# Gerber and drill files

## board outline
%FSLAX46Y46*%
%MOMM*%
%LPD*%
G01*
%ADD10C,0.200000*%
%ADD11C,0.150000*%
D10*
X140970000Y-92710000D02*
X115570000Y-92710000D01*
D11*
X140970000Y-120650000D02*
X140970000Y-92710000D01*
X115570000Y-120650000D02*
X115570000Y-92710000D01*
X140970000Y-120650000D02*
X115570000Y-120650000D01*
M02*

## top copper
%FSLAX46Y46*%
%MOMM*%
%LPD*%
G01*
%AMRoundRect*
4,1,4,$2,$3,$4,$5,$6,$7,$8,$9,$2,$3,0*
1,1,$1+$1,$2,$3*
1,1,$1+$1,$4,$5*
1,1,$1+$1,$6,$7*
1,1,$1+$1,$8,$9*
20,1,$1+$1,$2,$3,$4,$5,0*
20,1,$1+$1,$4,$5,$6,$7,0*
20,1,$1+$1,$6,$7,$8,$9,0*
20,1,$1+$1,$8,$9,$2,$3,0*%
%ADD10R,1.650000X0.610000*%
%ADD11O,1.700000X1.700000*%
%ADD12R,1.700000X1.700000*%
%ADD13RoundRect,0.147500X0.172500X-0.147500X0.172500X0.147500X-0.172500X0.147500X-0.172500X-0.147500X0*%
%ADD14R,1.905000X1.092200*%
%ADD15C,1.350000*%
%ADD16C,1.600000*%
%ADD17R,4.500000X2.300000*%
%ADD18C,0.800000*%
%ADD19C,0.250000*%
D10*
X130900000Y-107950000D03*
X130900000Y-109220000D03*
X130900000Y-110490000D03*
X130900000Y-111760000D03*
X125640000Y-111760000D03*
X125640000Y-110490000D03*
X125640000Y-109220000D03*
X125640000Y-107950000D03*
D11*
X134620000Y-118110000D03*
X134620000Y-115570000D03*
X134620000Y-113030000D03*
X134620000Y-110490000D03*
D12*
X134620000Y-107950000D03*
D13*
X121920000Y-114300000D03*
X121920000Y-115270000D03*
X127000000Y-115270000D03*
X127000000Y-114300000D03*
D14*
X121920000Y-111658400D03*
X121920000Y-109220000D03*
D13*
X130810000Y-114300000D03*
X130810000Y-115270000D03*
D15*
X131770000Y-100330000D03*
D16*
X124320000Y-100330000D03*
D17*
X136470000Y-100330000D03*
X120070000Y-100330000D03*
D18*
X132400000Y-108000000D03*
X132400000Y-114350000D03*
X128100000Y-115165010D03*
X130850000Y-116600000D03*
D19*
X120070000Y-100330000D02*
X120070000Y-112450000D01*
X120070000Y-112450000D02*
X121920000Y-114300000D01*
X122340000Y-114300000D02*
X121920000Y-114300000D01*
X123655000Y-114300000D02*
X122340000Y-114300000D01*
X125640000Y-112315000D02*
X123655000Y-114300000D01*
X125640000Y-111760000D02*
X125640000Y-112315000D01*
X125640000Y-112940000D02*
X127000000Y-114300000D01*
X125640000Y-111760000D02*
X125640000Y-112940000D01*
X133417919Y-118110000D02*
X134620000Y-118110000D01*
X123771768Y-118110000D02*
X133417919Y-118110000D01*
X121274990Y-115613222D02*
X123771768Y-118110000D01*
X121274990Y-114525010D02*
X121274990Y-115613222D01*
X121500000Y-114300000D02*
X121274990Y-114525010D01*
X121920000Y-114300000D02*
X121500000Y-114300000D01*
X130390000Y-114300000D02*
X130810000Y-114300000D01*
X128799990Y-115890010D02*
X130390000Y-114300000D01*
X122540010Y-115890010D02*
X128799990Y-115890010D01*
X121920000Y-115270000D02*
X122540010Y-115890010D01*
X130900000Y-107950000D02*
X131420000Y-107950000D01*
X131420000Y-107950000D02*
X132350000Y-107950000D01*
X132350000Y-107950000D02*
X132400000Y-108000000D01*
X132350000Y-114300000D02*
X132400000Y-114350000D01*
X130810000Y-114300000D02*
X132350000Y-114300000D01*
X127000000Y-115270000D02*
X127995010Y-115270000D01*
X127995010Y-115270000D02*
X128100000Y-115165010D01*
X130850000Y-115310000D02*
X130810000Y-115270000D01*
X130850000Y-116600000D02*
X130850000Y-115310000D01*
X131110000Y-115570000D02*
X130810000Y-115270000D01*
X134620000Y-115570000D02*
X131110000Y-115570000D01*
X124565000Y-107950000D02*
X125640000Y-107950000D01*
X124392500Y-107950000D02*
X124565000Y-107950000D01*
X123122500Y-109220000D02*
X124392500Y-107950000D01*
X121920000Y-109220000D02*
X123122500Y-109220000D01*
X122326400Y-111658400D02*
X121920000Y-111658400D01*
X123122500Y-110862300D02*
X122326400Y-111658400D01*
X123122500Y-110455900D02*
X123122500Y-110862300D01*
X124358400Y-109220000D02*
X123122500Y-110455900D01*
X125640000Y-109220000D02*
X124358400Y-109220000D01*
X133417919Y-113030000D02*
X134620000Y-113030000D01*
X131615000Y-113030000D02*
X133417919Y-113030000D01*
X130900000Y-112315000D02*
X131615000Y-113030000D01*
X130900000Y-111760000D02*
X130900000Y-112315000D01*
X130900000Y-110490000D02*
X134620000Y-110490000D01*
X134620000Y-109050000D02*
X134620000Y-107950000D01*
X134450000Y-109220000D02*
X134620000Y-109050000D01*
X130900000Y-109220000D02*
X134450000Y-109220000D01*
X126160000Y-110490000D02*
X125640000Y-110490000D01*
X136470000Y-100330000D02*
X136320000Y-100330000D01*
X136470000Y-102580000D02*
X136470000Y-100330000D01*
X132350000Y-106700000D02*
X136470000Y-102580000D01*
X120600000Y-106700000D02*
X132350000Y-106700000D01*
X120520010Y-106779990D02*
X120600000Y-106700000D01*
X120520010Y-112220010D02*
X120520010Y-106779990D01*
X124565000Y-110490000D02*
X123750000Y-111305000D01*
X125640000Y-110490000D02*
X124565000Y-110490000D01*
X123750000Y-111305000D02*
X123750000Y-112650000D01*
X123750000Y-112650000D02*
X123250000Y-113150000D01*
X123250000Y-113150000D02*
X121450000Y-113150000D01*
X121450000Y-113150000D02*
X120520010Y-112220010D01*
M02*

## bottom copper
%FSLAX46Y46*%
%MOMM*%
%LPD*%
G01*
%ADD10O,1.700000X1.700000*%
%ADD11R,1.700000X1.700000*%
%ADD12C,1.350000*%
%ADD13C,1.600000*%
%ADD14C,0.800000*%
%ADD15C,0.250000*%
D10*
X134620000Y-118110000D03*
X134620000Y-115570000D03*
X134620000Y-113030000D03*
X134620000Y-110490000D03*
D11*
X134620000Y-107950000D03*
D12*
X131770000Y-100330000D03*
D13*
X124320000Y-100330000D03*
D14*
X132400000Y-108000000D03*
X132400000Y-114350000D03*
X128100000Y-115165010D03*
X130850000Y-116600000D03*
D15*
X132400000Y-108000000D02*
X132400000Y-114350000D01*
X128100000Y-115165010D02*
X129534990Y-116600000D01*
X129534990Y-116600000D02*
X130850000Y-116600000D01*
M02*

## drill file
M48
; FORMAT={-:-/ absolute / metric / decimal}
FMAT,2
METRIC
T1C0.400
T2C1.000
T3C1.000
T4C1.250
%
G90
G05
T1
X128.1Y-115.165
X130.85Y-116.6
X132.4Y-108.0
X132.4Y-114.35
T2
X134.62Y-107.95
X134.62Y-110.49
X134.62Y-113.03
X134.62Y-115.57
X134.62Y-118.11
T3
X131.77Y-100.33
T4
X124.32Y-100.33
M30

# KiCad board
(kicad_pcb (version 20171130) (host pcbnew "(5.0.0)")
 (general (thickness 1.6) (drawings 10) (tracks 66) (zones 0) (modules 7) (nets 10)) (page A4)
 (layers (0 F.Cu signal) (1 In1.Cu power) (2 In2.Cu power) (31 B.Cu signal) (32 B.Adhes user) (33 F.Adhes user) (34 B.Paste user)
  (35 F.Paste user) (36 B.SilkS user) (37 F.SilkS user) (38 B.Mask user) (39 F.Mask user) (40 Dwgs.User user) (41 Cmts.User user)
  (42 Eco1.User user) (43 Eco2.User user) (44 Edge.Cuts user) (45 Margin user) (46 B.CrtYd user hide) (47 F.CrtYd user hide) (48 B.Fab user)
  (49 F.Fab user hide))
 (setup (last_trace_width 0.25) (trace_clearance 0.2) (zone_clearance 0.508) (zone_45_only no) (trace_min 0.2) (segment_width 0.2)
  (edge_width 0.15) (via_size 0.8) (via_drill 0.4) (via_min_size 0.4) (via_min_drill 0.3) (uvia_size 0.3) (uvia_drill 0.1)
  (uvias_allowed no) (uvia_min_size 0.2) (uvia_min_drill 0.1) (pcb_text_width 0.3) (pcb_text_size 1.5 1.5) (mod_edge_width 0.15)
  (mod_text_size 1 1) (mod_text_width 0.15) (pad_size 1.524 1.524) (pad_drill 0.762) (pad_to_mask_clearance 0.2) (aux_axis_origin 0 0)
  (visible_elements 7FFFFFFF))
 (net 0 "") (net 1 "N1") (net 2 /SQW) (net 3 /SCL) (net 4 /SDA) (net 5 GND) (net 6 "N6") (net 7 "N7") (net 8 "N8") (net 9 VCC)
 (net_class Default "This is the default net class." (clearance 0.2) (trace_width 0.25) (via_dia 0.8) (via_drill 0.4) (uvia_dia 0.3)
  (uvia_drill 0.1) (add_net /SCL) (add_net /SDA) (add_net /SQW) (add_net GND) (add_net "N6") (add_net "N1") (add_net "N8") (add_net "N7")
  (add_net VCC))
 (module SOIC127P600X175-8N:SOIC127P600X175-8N (layer F.Cu) (at 128.27 109.855)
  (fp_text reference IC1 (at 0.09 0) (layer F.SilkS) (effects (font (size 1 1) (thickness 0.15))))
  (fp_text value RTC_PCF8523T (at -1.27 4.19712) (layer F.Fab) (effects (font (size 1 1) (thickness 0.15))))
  (pad 8 smd rect (at 2.63 -1.905) (size 1.65 0.61) (layers F.Cu F.Paste F.Mask) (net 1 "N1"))
  (pad 7 smd rect (at 2.63 -0.635) (size 1.65 0.61) (layers F.Cu F.Paste F.Mask) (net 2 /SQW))
  (pad 6 smd rect (at 2.63 0.635) (size 1.65 0.61) (layers F.Cu F.Paste F.Mask) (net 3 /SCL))
  (pad 5 smd rect (at 2.63 1.905) (size 1.65 0.61) (layers F.Cu F.Paste F.Mask) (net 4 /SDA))
  (pad 4 smd rect (at -2.63 1.905) (size 1.65 0.61) (layers F.Cu F.Paste F.Mask) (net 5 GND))
  (pad 3 smd rect (at -2.63 0.635) (size 1.65 0.61) (layers F.Cu F.Paste F.Mask) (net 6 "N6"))
  (pad 2 smd rect (at -2.63 -0.635) (size 1.65 0.61) (layers F.Cu F.Paste F.Mask) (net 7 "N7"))
  (pad 1 smd rect (at -2.63 -1.905) (size 1.65 0.61) (layers F.Cu F.Paste F.Mask) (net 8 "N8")))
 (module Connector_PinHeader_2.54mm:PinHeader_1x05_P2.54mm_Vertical (layer F.Cu) (at 134.62 107.95)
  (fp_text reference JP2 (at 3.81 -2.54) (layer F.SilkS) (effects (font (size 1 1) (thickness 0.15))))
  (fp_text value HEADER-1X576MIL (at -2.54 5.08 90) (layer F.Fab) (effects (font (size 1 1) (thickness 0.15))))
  (pad 5 thru_hole oval (at 0 10.16) (size 1.7 1.7) (drill 1) (layers *.Cu *.Mask) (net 5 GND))
  (pad 4 thru_hole oval (at 0 7.62) (size 1.7 1.7) (drill 1) (layers *.Cu *.Mask) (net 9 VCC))
  (pad 3 thru_hole oval (at 0 5.08) (size 1.7 1.7) (drill 1) (layers *.Cu *.Mask) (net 4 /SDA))
  (pad 2 thru_hole oval (at 0 2.54) (size 1.7 1.7) (drill 1) (layers *.Cu *.Mask) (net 3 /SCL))
  (pad 1 thru_hole rect (at 0 0) (size 1.7 1.7) (drill 1) (layers *.Cu *.Mask) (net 2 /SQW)))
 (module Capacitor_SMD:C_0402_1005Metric (layer F.Cu) (at 121.92 114.785 90)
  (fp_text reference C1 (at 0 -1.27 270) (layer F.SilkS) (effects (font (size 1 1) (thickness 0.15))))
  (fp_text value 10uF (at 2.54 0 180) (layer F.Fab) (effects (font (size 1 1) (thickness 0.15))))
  (pad 2 smd roundrect (at 0.485 0 90) (size 0.59 0.64) (layers F.Cu F.Paste F.Mask) (roundrect_rratio 0.25) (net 5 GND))
  (pad 1 smd roundrect (at -0.485 0 90) (size 0.59 0.64) (layers F.Cu F.Paste F.Mask) (roundrect_rratio 0.25) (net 1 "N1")))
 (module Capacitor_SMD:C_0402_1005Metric (layer F.Cu) (at 127 114.785 90)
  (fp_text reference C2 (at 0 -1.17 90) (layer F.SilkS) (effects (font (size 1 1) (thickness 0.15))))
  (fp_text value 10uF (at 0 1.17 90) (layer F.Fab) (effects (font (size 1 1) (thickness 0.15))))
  (pad 1 smd roundrect (at -0.485 0 90) (size 0.59 0.64) (layers F.Cu F.Paste F.Mask) (roundrect_rratio 0.25) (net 9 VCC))
  (pad 2 smd roundrect (at 0.485 0 90) (size 0.59 0.64) (layers F.Cu F.Paste F.Mask) (roundrect_rratio 0.25) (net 5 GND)))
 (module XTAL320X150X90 (layer F.Cu) (at 121.92 110.4392 270)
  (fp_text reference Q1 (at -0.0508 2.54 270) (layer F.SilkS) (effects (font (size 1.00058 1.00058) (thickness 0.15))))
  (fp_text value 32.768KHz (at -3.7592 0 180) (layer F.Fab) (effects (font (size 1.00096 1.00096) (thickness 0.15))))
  (pad 2 smd rect (at 1.2192 0 270) (size 1.0922 1.905) (layers F.Cu F.Paste F.Mask) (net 7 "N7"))
  (pad 1 smd rect (at -1.2192 0 270) (size 1.0922 1.905) (layers F.Cu F.Paste F.Mask) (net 8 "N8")))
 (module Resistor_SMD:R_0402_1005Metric (layer F.Cu) (at 130.81 114.785 90)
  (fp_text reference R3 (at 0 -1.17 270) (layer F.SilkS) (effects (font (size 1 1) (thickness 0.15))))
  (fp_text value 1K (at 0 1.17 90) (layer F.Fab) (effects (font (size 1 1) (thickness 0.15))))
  (pad 2 smd roundrect (at 0.485 0 90) (size 0.59 0.64) (layers F.Cu F.Paste F.Mask) (roundrect_rratio 0.25) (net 1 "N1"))
  (pad 1 smd roundrect (at -0.485 0 90) (size 0.59 0.64) (layers F.Cu F.Paste F.Mask) (roundrect_rratio 0.25) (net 9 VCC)))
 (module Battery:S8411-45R (layer F.Cu) (at 128.27 100.33 270)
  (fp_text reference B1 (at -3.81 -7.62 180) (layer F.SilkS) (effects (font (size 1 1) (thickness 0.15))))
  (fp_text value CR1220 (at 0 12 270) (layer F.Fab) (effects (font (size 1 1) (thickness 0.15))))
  (pad "" np_thru_hole circle (at 0 -3.5 270) (size 1.35 1.35) (drill 1) (layers *.Cu *.Mask))
  (pad "" np_thru_hole circle (at 0 3.95 270) (size 1.6 1.6) (drill 1.25) (layers *.Cu *.Mask))
  (pad 2 smd rect (at 0 -8.2 270) (size 2.3 4.5) (layers F.Cu F.Paste F.Mask) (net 6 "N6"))
  (pad 1 smd rect (at 0 8.2 270) (size 2.3 4.5) (layers F.Cu F.Paste F.Mask) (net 5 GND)))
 (gr_line (start 140.97 92.71) (end 115.57 92.71) (layer Edge.Cuts) (width 0.2))
 (gr_line (start 140.97 120.65) (end 140.97 92.71) (layer Edge.Cuts) (width 0.15))
 (gr_line (start 115.57 120.65) (end 115.57 92.71) (layer Edge.Cuts) (width 0.15))
 (gr_line (start 140.97 120.65) (end 115.57 120.65) (layer Edge.Cuts) (width 0.15))
 (segment (start 120.07 100.33) (end 120.07 112.45) (width 0.25) (layer F.Cu) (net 5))
 (segment (start 120.07 112.45) (end 121.92 114.3) (width 0.25) (layer F.Cu) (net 5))
 (segment (start 122.34 114.3) (end 121.92 114.3) (width 0.25) (layer F.Cu) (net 5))
 (segment (start 123.655 114.3) (end 122.34 114.3) (width 0.25) (layer F.Cu) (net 5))
 (segment (start 125.64 112.315) (end 123.655 114.3) (width 0.25) (layer F.Cu) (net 5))
 (segment (start 125.64 111.76) (end 125.64 112.315) (width 0.25) (layer F.Cu) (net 5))
 (segment (start 125.64 112.94) (end 127 114.3) (width 0.25) (layer F.Cu) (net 5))
 (segment (start 125.64 111.76) (end 125.64 112.94) (width 0.25) (layer F.Cu) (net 5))
 (segment (start 133.417919 118.11) (end 134.62 118.11) (width 0.25) (layer F.Cu) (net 5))
 (segment (start 123.771768 118.11) (end 133.417919 118.11) (width 0.25) (layer F.Cu) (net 5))
 (segment (start 121.27499 115.613222) (end 123.771768 118.11) (width 0.25) (layer F.Cu) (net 5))
 (segment (start 121.27499 114.52501) (end 121.27499 115.613222) (width 0.25) (layer F.Cu) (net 5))
 (segment (start 121.5 114.3) (end 121.27499 114.52501) (width 0.25) (layer F.Cu) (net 5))
 (segment (start 121.92 114.3) (end 121.5 114.3) (width 0.25) (layer F.Cu) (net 5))
 (segment (start 130.39 114.3) (end 130.81 114.3) (width 0.25) (layer F.Cu) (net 1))
 (segment (start 128.79999 115.89001) (end 130.39 114.3) (width 0.25) (layer F.Cu) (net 1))
 (segment (start 122.54001 115.89001) (end 128.79999 115.89001) (width 0.25) (layer F.Cu) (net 1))
 (segment (start 121.92 115.27) (end 122.54001 115.89001) (width 0.25) (layer F.Cu) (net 1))
 (segment (start 130.9 107.95) (end 131.42 107.95) (width 0.25) (layer F.Cu) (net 1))
 (via (at 132.4 108) (size 0.8) (drill 0.4) (layers F.Cu B.Cu) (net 1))
 (segment (start 131.42 107.95) (end 132.35 107.95) (width 0.25) (layer F.Cu) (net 1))
 (segment (start 132.35 107.95) (end 132.4 108) (width 0.25) (layer F.Cu) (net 1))
 (segment (start 132.4 108) (end 132.4 114.35) (width 0.25) (layer B.Cu) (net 1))
 (via (at 132.4 114.35) (size 0.8) (drill 0.4) (layers F.Cu B.Cu) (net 1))
 (segment (start 132.35 114.3) (end 132.4 114.35) (width 0.25) (layer F.Cu) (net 1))
 (segment (start 130.81 114.3) (end 132.35 114.3) (width 0.25) (layer F.Cu) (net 1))
 (via (at 128.1 115.16501) (size 0.8) (drill 0.4) (layers F.Cu B.Cu) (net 9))
 (segment (start 127 115.27) (end 127.99501 115.27) (width 0.25) (layer F.Cu) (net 9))
 (segment (start 127.99501 115.27) (end 128.1 115.16501) (width 0.25) (layer F.Cu) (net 9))
 (segment (start 128.1 115.16501) (end 129.53499 116.6) (width 0.25) (layer B.Cu) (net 9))
 (via (at 130.85 116.6) (size 0.8) (drill 0.4) (layers F.Cu B.Cu) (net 9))
 (segment (start 129.53499 116.6) (end 130.85 116.6) (width 0.25) (layer B.Cu) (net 9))
 (segment (start 130.85 115.31) (end 130.81 115.27) (width 0.25) (layer F.Cu) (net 9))
 (segment (start 130.85 116.6) (end 130.85 115.31) (width 0.25) (layer F.Cu) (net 9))
 (segment (start 131.11 115.57) (end 130.81 115.27) (width 0.25) (layer F.Cu) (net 9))
 (segment (start 134.62 115.57) (end 131.11 115.57) (width 0.25) (layer F.Cu) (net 9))
 (segment (start 124.565 107.95) (end 125.64 107.95) (width 0.25) (layer F.Cu) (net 8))
 (segment (start 124.3925 107.95) (end 124.565 107.95) (width 0.25) (layer F.Cu) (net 8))
 (segment (start 123.1225 109.22) (end 124.3925 107.95) (width 0.25) (layer F.Cu) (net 8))
 (segment (start 121.92 109.22) (end 123.1225 109.22) (width 0.25) (layer F.Cu) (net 8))
 (segment (start 122.3264 111.6584) (end 121.92 111.6584) (width 0.25) (layer F.Cu) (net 7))
 (segment (start 123.1225 110.8623) (end 122.3264 111.6584) (width 0.25) (layer F.Cu) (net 7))
 (segment (start 123.1225 110.4559) (end 123.1225 110.8623) (width 0.25) (layer F.Cu) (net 7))
 (segment (start 124.3584 109.22) (end 123.1225 110.4559) (width 0.25) (layer F.Cu) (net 7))
 (segment (start 125.64 109.22) (end 124.3584 109.22) (width 0.25) (layer F.Cu) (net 7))
 (segment (start 133.417919 113.03) (end 134.62 113.03) (width 0.25) (layer F.Cu) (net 4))
 (segment (start 131.615 113.03) (end 133.417919 113.03) (width 0.25) (layer F.Cu) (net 4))
 (segment (start 130.9 112.315) (end 131.615 113.03) (width 0.25) (layer F.Cu) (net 4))
 (segment (start 130.9 111.76) (end 130.9 112.315) (width 0.25) (layer F.Cu) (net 4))
 (segment (start 130.9 110.49) (end 134.62 110.49) (width 0.25) (layer F.Cu) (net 3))
 (segment (start 134.62 109.05) (end 134.62 107.95) (width 0.25) (layer F.Cu) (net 2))
 (segment (start 134.45 109.22) (end 134.62 109.05) (width 0.25) (layer F.Cu) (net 2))
 (segment (start 130.9 109.22) (end 134.45 109.22) (width 0.25) (layer F.Cu) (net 2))
 (segment (start 126.16 110.49) (end 125.64 110.49) (width 0.25) (layer F.Cu) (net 6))
 (segment (start 136.47 100.33) (end 136.32 100.33) (width 0.25) (layer F.Cu) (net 6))
 (segment (start 136.47 102.58) (end 136.47 100.33) (width 0.25) (layer F.Cu) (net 6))
 (segment (start 132.35 106.7) (end 136.47 102.58) (width 0.25) (layer F.Cu) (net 6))
 (segment (start 120.6 106.7) (end 132.35 106.7) (width 0.25) (layer F.Cu) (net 6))
 (segment (start 120.52001 106.77999) (end 120.6 106.7) (width 0.25) (layer F.Cu) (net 6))
 (segment (start 120.52001 112.22001) (end 120.52001 106.77999) (width 0.25) (layer F.Cu) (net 6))
 (segment (start 124.565 110.49) (end 123.75 111.305) (width 0.25) (layer F.Cu) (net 6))
 (segment (start 125.64 110.49) (end 124.565 110.49) (width 0.25) (layer F.Cu) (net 6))
 (segment (start 123.75 111.305) (end 123.75 112.65) (width 0.25) (layer F.Cu) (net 6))
 (segment (start 123.75 112.65) (end 123.25 113.15) (width 0.25) (layer F.Cu) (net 6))
 (segment (start 123.25 113.15) (end 121.45 113.15) (width 0.25) (layer F.Cu) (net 6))
 (segment (start 121.45 113.15) (end 120.52001 112.22001) (width 0.25) (layer F.Cu) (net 6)))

